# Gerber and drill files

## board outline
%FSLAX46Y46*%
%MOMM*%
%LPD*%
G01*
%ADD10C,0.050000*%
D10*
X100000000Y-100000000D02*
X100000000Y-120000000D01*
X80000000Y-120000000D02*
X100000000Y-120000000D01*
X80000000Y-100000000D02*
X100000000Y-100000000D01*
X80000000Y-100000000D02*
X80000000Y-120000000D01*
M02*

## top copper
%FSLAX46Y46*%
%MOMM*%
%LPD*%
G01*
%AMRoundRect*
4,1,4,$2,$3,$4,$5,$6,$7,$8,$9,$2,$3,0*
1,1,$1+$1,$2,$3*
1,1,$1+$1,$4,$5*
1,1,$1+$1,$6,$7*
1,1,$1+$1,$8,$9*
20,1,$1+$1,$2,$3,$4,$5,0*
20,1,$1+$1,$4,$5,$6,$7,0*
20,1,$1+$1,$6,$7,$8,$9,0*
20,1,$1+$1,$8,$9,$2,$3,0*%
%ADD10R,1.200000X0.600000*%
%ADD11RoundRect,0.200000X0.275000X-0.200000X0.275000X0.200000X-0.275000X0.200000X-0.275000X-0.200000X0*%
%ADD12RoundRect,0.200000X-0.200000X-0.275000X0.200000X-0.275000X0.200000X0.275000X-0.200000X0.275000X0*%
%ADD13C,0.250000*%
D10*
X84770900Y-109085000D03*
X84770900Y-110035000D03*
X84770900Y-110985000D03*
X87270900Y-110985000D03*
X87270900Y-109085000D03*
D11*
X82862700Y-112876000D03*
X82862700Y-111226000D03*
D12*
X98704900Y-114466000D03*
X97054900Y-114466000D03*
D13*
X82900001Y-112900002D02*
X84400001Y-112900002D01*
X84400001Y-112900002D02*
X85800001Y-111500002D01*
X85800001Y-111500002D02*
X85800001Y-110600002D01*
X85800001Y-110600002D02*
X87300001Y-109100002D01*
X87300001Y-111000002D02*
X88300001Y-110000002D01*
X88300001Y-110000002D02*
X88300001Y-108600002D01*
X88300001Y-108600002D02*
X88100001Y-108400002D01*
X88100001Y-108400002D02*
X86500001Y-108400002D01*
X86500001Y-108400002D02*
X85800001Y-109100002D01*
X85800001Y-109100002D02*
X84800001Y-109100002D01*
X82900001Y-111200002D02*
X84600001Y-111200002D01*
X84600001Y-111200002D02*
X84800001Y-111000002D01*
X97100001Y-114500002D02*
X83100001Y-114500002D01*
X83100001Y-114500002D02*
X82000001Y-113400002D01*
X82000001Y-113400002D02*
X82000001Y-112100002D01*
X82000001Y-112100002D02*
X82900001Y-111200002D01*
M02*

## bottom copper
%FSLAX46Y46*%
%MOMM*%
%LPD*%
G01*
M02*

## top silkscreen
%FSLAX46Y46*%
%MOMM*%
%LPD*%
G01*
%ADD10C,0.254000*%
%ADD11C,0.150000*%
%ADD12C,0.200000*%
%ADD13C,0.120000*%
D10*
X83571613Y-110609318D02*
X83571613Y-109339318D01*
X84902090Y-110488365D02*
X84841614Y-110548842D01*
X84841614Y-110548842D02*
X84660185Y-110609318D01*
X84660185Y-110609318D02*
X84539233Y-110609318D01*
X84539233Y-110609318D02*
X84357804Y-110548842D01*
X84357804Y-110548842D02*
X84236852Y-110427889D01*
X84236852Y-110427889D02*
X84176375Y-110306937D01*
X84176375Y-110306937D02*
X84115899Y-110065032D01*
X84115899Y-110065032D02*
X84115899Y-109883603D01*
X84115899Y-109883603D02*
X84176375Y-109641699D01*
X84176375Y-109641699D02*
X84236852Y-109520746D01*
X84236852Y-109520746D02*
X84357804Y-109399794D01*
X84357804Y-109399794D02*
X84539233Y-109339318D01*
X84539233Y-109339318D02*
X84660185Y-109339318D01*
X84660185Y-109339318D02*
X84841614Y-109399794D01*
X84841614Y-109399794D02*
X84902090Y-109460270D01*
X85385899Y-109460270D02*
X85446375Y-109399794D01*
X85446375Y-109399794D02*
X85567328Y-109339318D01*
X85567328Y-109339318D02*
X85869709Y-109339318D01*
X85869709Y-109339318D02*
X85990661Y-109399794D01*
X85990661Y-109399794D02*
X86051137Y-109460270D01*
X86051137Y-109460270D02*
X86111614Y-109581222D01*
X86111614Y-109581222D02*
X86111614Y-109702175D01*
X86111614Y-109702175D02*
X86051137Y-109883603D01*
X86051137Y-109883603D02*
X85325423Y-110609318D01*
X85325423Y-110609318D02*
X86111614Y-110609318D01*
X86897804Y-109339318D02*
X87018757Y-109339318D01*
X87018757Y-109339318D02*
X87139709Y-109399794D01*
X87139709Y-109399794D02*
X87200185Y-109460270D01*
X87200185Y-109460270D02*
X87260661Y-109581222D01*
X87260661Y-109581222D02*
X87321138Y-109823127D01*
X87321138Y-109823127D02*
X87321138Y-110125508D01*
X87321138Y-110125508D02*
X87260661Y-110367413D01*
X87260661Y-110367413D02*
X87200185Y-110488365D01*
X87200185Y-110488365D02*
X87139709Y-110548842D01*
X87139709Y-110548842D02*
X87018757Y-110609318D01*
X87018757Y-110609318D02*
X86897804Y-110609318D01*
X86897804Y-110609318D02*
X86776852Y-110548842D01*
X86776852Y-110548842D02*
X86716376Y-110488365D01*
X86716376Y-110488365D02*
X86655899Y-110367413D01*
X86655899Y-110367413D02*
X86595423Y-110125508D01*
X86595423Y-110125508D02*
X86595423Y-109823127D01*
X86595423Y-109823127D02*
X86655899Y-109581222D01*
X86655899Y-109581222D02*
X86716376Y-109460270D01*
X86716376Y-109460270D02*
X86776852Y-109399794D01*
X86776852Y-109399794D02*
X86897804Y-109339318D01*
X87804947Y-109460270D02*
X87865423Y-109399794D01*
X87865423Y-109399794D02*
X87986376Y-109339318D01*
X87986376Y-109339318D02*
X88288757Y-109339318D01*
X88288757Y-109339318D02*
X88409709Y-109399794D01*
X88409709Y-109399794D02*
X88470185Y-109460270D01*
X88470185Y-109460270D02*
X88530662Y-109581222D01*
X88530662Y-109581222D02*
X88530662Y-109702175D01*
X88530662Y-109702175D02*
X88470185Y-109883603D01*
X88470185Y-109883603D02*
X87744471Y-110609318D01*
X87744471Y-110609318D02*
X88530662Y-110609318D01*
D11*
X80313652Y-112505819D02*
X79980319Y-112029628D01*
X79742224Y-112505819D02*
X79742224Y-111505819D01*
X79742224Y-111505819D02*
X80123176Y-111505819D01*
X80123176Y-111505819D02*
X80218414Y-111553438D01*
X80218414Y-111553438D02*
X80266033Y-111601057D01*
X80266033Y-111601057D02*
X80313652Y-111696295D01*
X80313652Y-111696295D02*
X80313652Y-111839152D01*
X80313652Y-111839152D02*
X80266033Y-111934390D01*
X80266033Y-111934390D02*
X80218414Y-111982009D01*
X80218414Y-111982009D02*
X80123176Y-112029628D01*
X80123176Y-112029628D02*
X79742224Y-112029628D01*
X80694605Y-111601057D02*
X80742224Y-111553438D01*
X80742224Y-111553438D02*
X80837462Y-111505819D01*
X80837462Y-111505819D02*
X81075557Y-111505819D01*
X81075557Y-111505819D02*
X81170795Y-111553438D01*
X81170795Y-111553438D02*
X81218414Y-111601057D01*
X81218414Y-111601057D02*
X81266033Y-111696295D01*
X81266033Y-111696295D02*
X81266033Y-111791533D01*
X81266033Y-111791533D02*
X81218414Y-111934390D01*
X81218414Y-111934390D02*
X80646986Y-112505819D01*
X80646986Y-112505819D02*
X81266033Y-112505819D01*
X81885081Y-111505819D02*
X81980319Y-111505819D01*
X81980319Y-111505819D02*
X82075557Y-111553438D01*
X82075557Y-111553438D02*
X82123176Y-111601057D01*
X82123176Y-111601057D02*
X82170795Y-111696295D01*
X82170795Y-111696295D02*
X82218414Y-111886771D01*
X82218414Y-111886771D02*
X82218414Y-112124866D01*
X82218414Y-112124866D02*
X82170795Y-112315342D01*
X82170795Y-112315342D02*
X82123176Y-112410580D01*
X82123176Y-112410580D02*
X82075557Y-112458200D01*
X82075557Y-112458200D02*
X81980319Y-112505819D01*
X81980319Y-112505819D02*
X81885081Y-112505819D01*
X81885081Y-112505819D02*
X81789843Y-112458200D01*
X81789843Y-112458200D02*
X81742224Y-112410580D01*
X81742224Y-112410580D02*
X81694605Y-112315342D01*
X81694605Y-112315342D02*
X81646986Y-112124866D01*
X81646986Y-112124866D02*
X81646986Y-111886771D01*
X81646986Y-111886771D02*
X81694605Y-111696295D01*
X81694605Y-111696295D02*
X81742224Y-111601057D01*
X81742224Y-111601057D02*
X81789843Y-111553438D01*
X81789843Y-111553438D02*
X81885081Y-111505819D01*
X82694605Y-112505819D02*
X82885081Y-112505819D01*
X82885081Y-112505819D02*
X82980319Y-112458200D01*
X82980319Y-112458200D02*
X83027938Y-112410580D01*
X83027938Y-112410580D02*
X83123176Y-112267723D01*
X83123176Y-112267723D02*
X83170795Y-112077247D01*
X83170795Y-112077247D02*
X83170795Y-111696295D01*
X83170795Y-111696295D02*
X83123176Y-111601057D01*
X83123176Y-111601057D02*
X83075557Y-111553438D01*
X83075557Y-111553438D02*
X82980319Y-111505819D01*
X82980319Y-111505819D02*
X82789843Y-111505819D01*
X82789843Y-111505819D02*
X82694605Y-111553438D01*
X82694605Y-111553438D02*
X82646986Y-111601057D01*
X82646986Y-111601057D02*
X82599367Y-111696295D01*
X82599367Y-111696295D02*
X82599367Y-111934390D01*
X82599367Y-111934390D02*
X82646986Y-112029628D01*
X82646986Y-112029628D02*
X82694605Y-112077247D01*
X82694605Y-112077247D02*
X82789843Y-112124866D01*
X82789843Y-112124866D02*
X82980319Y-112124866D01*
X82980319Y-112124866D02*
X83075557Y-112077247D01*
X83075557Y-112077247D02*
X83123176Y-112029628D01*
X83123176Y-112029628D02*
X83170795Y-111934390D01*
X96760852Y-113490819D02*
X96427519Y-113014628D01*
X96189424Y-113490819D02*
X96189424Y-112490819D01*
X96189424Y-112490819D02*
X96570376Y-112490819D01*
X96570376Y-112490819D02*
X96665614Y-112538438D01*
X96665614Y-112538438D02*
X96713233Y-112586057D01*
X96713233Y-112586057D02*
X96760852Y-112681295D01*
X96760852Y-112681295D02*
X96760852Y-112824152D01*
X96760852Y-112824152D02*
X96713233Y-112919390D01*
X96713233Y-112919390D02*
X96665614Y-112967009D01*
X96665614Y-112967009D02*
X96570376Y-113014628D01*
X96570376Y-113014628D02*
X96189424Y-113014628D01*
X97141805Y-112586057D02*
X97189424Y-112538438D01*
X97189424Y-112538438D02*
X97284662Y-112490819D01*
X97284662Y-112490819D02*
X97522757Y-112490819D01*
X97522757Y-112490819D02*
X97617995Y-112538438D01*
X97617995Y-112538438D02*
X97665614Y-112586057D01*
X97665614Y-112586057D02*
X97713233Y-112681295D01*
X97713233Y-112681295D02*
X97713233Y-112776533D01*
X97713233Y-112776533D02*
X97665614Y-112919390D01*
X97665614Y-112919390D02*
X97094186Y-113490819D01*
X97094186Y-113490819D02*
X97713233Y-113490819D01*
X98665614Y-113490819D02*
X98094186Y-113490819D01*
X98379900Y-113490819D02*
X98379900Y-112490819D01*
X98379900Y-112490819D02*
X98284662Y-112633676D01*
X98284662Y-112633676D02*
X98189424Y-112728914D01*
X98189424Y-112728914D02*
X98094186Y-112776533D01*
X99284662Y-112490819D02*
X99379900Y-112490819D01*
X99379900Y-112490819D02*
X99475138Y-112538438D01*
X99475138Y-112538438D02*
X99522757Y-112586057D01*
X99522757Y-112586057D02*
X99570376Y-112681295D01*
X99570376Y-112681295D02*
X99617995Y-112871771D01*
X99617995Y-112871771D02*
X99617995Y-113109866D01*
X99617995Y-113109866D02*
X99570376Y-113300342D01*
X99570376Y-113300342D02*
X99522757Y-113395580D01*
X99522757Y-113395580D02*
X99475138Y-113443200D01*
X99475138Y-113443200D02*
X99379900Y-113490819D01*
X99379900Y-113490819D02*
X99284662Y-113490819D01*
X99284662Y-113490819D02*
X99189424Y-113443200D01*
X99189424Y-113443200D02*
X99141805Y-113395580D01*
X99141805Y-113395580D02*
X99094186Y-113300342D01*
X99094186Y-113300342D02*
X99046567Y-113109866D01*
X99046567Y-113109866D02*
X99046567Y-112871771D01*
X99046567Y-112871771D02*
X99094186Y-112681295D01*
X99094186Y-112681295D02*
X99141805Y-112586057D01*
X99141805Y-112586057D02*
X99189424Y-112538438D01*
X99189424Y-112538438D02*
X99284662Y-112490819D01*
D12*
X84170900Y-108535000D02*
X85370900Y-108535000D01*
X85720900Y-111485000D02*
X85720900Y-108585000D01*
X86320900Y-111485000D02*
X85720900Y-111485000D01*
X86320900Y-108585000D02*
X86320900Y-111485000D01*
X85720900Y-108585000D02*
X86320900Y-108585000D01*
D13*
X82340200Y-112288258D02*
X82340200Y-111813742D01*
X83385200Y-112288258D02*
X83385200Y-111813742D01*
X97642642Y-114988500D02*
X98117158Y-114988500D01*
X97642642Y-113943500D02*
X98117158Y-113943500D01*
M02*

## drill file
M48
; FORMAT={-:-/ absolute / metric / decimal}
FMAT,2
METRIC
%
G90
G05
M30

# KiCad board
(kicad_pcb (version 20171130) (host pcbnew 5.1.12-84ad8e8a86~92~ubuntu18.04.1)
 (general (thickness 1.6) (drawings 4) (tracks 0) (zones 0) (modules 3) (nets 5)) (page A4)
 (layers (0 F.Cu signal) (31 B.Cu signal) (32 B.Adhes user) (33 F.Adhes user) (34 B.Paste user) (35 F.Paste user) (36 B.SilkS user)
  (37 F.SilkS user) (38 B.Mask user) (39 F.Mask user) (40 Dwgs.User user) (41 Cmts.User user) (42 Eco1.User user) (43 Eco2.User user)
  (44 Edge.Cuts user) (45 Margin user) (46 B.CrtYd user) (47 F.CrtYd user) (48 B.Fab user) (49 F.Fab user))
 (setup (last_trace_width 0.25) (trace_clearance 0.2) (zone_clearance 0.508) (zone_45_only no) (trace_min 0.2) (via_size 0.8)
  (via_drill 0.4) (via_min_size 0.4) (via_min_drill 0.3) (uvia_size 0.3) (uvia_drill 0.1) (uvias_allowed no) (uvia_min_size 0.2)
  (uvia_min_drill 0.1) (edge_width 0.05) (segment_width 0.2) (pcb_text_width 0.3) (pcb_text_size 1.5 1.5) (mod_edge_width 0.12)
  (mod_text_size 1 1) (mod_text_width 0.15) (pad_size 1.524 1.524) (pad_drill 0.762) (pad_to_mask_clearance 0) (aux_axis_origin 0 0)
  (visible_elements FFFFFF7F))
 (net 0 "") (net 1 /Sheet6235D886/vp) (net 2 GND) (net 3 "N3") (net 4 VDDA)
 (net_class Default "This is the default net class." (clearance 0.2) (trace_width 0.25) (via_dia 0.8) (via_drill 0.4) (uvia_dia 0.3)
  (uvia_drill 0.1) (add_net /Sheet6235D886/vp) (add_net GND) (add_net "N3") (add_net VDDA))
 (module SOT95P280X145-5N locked (layer F.Cu) (at 86.020900 110.035000)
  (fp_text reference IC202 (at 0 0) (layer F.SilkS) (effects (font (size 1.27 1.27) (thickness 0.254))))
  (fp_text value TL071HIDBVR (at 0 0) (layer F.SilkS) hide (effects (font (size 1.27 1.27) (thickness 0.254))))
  (fp_line (start -1.85 -1.5) (end -0.65 -1.5) (layer F.SilkS) (width 0.2))
  (fp_line (start -0.3 1.45) (end -0.3 -1.45) (layer F.SilkS) (width 0.2))
  (fp_line (start 0.3 1.45) (end -0.3 1.45) (layer F.SilkS) (width 0.2))
  (fp_line (start 0.3 -1.45) (end 0.3 1.45) (layer F.SilkS) (width 0.2))
  (fp_line (start -0.3 -1.45) (end 0.3 -1.45) (layer F.SilkS) (width 0.2))
  (pad 1 smd rect (at -1.25 -0.95 90.000000) (size 0.6 1.2) (layers F.Cu F.Mask F.Paste) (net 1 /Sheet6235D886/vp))
  (pad 2 smd rect (at -1.25 0 90.000000) (size 0.6 1.2) (layers F.Cu F.Mask F.Paste) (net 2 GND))
  (pad 3 smd rect (at -1.25 0.95 90.000000) (size 0.6 1.2) (layers F.Cu F.Mask F.Paste) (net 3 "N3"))
  (pad 4 smd rect (at 1.25 0.95 90.000000) (size 0.6 1.2) (layers F.Cu F.Mask F.Paste) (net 1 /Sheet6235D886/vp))
  (pad 5 smd rect (at 1.25 -0.95 90.000000) (size 0.6 1.2) (layers F.Cu F.Mask F.Paste) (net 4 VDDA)))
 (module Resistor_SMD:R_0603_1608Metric (layer F.Cu) (at 82.862700 112.051000 90.000000)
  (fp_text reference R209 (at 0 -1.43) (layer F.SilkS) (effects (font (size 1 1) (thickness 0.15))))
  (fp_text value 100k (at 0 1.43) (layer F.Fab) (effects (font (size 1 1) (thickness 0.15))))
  (fp_line (start -0.237258 -0.5225) (end 0.237258 -0.5225) (layer F.SilkS) (width 0.12))
  (fp_line (start -0.237258 0.5225) (end 0.237258 0.5225) (layer F.SilkS) (width 0.12))
  (pad 1 smd roundrect (at -0.825 0 90.000000) (size 0.8 0.95) (layers F.Cu F.Mask F.Paste) (roundrect_rratio 0.25) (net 4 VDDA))
  (pad 2 smd roundrect (at 0.825 0 90.000000) (size 0.8 0.95) (layers F.Cu F.Mask F.Paste) (roundrect_rratio 0.25) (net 3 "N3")))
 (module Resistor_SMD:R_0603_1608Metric (layer F.Cu) (at 97.879900 114.466000)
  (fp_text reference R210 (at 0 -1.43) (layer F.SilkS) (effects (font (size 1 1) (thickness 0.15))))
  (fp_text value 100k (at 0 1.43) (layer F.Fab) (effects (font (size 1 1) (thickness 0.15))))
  (fp_line (start -0.237258 0.5225) (end 0.237258 0.5225) (layer F.SilkS) (width 0.12))
  (fp_line (start -0.237258 -0.5225) (end 0.237258 -0.5225) (layer F.SilkS) (width 0.12))
  (pad 2 smd roundrect (at 0.825 0) (size 0.8 0.95) (layers F.Cu F.Mask F.Paste) (roundrect_rratio 0.25) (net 2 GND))
  (pad 1 smd roundrect (at -0.825 0) (size 0.8 0.95) (layers F.Cu F.Mask F.Paste) (roundrect_rratio 0.25) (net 3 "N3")))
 (gr_line (start 100 100) (end 100 120) (layer Edge.Cuts) (width 0.05))
 (gr_line (start 80 120) (end 100 120) (layer Edge.Cuts) (width 0.05))
 (gr_line (start 80 100) (end 100 100) (layer Edge.Cuts) (width 0.05))
 (gr_line (start 80 100) (end 80 120) (layer Edge.Cuts) (width 0.05))
 (segment (start 82.900001 112.900002) (end 84.400001 112.900002) (width 0.250000) (layer F.Cu) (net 4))
 (segment (start 84.400001 112.900002) (end 85.800001 111.500002) (width 0.250000) (layer F.Cu) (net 4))
 (segment (start 85.800001 111.500002) (end 85.800001 110.600002) (width 0.250000) (layer F.Cu) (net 4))
 (segment (start 85.800001 110.600002) (end 87.300001 109.100002) (width 0.250000) (layer F.Cu) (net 4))
 (segment (start 87.300001 111.000002) (end 88.300001 110.000002) (width 0.250000) (layer F.Cu) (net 1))
 (segment (start 88.300001 110.000002) (end 88.300001 108.600002) (width 0.250000) (layer F.Cu) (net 1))
 (segment (start 88.300001 108.600002) (end 88.100001 108.400002) (width 0.250000) (layer F.Cu) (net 1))
 (segment (start 88.100001 108.400002) (end 86.500001 108.400002) (width 0.250000) (layer F.Cu) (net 1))
 (segment (start 86.500001 108.400002) (end 85.800001 109.100002) (width 0.250000) (layer F.Cu) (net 1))
 (segment (start 85.800001 109.100002) (end 84.800001 109.100002) (width 0.250000) (layer F.Cu) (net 1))
 (segment (start 82.900001 111.200002) (end 84.600001 111.200002) (width 0.250000) (layer F.Cu) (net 3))
 (segment (start 84.600001 111.200002) (end 84.800001 111.000002) (width 0.250000) (layer F.Cu) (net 3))
 (segment (start 97.100001 114.500002) (end 83.100001 114.500002) (width 0.250000) (layer F.Cu) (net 3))
 (segment (start 83.100001 114.500002) (end 82.000001 113.400002) (width 0.250000) (layer F.Cu) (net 3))
 (segment (start 82.000001 113.400002) (end 82.000001 112.100002) (width 0.250000) (layer F.Cu) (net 3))
 (segment (start 82.000001 112.100002) (end 82.900001 111.200002) (width 0.250000) (layer F.Cu) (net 3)))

